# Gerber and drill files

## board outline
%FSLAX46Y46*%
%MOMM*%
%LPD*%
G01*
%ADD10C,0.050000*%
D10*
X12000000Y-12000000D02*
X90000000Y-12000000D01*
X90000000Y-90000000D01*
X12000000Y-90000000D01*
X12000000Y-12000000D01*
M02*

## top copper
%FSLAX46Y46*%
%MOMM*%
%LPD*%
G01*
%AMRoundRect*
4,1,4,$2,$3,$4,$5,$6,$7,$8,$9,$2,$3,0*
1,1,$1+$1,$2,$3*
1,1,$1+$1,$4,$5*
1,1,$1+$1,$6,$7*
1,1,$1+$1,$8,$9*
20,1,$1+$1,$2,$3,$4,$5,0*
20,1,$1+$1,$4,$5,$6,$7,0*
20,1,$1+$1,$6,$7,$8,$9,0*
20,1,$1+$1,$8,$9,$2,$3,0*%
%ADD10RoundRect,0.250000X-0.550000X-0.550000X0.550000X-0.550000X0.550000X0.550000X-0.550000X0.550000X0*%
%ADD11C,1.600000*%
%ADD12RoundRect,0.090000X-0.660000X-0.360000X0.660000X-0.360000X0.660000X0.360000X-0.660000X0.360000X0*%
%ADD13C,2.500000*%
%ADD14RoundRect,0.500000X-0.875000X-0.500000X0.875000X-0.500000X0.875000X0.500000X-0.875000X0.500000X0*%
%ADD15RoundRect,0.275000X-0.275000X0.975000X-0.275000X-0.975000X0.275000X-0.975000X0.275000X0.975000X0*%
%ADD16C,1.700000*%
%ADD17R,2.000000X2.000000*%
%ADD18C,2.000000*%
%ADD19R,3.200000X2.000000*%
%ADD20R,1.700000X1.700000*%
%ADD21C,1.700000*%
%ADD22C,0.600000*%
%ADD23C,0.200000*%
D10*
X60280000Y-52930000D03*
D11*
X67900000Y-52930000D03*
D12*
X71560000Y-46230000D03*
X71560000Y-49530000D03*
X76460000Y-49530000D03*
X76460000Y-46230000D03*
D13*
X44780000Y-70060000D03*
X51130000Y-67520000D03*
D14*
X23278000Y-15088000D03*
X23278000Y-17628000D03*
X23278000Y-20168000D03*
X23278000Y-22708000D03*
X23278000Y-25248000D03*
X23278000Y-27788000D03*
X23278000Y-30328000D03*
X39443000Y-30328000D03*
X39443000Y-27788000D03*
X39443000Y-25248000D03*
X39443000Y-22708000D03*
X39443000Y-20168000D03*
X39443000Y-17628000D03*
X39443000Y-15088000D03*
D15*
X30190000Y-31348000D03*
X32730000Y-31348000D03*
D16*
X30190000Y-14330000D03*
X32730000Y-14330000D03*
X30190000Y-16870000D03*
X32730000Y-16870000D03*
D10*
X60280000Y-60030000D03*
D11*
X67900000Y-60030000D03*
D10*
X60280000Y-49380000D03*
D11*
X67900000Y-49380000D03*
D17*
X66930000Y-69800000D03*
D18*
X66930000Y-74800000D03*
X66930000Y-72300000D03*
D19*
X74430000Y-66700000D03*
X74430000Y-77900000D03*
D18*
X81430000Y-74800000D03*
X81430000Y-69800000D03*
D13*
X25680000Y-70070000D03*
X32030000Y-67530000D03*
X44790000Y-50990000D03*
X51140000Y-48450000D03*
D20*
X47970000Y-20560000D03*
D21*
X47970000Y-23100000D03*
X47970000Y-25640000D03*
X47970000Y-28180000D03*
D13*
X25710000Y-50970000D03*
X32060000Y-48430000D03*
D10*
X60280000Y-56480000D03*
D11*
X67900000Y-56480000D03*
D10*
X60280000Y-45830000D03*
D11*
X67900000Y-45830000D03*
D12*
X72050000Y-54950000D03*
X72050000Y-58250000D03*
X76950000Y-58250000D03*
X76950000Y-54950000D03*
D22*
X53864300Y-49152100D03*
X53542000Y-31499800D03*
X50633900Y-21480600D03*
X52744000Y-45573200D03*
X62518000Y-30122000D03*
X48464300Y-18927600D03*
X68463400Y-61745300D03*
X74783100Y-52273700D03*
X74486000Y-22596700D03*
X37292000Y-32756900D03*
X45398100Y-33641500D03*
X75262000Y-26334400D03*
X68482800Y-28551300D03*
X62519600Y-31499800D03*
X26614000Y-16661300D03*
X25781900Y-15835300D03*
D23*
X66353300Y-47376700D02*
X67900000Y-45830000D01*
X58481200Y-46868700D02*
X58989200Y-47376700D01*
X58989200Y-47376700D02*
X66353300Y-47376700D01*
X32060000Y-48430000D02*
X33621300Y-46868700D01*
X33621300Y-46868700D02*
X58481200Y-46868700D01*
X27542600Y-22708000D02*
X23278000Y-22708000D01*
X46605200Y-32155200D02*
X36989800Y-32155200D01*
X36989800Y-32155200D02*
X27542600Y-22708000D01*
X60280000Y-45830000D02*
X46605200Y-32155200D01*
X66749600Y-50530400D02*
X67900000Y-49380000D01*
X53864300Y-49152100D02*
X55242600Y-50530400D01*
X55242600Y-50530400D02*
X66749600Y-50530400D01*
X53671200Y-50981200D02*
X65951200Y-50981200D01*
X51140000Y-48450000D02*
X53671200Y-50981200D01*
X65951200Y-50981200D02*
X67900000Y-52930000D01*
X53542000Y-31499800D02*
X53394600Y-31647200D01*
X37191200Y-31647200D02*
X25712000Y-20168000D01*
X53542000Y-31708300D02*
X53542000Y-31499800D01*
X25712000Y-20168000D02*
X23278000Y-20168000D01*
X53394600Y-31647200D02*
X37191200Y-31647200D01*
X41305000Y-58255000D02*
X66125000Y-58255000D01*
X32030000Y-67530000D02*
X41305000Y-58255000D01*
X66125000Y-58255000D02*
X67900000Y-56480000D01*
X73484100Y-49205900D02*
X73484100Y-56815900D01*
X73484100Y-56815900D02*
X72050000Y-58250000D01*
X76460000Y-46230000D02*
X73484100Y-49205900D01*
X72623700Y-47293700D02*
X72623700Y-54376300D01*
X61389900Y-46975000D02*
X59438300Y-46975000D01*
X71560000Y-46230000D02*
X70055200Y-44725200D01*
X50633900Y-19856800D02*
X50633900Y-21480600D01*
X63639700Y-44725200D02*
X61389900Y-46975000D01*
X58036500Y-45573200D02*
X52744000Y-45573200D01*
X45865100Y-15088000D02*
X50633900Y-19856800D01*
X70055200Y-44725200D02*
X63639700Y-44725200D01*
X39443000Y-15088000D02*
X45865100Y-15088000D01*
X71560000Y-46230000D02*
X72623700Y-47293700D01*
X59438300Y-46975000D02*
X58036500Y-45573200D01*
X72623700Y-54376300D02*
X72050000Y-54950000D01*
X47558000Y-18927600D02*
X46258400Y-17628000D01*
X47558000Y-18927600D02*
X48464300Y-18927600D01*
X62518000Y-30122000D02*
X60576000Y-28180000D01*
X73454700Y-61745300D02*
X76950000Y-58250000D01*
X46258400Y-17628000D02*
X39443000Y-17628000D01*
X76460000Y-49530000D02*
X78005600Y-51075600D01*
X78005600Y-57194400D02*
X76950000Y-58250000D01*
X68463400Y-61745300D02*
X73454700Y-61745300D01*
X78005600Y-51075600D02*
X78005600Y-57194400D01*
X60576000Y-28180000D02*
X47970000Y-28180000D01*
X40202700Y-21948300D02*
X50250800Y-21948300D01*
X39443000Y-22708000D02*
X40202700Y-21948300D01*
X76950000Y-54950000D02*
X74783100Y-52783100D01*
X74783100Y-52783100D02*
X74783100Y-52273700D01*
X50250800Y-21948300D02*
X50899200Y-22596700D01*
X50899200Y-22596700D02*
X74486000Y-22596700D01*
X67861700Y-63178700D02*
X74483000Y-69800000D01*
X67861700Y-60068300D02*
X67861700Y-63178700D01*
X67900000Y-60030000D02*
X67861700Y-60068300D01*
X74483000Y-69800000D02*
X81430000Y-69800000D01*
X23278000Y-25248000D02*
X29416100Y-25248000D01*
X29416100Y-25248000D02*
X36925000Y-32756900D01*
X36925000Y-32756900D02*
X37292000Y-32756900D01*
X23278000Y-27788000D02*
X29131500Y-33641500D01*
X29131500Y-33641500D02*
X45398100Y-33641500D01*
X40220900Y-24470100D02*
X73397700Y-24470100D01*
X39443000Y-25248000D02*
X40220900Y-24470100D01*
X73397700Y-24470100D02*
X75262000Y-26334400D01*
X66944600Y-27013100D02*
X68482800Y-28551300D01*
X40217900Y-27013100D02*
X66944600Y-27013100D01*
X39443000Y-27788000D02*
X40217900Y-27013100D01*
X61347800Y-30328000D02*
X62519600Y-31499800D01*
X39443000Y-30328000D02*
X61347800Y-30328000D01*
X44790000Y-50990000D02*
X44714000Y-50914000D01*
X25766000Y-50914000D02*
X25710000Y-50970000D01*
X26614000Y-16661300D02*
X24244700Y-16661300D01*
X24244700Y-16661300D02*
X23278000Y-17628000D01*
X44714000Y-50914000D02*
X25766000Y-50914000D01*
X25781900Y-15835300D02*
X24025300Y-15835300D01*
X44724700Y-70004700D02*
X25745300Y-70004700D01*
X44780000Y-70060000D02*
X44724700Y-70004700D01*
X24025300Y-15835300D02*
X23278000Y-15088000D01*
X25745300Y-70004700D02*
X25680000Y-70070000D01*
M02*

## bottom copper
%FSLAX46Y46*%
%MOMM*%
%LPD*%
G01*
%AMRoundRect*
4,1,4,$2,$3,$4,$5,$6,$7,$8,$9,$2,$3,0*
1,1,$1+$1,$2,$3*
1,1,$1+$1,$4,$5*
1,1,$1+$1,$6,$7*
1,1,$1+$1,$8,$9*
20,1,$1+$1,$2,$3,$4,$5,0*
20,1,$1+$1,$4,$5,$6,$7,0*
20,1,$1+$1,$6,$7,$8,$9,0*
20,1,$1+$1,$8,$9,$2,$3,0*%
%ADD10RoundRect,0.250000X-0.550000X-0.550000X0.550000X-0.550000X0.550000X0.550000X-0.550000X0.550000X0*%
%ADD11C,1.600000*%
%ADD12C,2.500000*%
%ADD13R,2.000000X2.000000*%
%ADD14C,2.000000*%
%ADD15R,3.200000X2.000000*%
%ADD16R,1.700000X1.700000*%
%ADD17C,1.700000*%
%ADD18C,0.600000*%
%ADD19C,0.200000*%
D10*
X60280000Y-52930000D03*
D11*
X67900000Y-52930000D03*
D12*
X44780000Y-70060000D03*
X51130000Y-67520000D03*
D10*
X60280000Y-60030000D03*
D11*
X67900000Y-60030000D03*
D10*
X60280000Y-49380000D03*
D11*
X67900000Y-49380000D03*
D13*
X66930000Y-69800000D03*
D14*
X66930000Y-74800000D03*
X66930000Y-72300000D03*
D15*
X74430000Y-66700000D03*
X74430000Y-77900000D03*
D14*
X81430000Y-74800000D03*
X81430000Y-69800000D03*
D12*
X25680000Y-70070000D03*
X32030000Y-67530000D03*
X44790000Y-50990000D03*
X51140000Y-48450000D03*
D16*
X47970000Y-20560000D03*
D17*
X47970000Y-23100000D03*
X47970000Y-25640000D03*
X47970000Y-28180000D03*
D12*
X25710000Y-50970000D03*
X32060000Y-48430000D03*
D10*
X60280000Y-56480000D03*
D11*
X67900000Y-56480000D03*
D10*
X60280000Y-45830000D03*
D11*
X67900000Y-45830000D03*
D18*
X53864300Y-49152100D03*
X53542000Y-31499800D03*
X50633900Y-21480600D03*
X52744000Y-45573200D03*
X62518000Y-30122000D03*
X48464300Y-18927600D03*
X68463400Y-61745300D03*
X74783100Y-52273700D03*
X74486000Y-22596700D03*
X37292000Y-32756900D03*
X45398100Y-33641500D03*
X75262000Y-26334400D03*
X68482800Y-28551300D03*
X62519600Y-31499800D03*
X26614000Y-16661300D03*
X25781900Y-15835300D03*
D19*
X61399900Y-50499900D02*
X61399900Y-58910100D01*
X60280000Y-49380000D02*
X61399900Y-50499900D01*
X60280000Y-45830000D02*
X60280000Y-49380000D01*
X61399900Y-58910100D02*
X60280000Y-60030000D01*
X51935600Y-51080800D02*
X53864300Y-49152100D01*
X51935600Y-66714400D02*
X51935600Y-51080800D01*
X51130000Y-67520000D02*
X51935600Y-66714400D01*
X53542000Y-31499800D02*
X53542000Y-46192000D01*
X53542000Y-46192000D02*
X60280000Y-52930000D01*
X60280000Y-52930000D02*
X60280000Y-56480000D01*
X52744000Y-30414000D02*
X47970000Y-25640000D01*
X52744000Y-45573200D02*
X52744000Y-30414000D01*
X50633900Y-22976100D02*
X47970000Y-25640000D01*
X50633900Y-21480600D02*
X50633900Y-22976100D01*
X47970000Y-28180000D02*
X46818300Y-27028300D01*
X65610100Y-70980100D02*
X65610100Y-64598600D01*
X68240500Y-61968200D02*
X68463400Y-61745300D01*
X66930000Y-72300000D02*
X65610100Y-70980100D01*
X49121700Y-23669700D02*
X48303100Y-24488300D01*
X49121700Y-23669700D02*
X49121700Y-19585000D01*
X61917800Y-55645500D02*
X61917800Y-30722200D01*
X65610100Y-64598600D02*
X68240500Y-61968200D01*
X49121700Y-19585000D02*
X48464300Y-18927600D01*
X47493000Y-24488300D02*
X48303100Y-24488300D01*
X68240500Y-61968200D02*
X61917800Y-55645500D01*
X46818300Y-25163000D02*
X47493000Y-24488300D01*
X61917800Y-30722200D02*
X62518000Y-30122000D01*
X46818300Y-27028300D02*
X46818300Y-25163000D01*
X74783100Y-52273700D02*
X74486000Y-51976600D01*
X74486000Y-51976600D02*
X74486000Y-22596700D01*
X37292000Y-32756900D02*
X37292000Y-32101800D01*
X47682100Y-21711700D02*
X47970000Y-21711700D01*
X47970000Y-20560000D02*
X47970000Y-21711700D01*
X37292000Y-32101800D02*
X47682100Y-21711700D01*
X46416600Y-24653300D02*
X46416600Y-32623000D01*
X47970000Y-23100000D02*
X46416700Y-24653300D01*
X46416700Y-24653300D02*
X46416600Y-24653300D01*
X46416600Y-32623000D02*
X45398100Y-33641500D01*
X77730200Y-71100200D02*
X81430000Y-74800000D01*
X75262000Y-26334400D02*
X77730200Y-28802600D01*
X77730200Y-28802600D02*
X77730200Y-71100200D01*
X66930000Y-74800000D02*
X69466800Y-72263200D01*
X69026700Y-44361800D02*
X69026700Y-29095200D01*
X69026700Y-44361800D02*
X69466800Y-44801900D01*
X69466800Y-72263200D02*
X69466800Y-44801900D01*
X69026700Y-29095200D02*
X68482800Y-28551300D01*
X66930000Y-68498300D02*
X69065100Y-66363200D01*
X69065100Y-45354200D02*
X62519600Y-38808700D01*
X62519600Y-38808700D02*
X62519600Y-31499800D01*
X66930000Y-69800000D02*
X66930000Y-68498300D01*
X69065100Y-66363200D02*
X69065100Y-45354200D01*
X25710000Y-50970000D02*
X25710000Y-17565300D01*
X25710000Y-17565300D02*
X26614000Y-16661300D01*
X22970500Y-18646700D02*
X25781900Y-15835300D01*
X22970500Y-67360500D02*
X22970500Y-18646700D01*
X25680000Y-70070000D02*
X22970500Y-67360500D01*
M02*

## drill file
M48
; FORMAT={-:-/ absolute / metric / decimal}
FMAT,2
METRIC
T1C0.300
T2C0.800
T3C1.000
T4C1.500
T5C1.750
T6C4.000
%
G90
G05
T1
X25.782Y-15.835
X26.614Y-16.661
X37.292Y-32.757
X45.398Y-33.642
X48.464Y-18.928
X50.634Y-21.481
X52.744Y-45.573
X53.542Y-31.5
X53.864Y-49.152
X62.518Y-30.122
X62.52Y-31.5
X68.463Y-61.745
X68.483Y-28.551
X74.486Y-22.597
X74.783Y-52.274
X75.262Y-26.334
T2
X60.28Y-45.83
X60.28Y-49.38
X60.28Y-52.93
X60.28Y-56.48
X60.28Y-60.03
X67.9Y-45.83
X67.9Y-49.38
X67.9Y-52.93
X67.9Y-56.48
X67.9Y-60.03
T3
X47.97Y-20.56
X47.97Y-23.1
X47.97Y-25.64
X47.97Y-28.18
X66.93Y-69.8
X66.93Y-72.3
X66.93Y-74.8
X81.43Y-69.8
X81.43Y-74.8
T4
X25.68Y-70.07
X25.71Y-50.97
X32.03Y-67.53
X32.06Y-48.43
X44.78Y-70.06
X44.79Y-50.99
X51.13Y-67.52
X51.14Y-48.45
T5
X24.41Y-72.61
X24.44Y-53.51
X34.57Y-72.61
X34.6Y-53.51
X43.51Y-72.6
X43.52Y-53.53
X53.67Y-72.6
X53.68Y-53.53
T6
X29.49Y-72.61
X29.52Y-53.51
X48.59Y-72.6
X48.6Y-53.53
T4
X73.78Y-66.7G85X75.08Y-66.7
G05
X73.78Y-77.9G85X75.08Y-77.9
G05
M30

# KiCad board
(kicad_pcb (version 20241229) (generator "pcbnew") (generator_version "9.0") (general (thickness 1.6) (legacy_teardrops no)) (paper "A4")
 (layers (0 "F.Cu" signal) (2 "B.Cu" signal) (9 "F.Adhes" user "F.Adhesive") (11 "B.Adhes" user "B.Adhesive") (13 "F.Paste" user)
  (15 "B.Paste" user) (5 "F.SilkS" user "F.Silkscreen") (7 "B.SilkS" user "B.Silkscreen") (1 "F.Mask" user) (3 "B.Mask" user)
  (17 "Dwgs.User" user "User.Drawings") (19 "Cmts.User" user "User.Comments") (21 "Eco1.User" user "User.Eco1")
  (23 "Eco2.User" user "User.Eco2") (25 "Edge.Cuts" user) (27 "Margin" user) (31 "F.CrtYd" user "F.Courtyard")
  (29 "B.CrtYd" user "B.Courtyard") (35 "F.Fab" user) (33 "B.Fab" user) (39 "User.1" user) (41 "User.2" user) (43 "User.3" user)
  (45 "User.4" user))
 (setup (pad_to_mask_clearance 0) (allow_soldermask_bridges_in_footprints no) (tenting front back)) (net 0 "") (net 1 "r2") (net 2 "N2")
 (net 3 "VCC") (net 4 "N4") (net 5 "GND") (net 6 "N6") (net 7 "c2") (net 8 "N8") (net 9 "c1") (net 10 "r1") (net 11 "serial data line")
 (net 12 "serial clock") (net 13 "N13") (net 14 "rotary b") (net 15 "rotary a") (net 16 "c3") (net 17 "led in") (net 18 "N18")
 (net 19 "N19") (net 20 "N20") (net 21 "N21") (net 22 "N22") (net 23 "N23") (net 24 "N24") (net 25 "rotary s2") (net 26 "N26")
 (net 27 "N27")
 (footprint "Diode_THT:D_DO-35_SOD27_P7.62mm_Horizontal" (layer "F.Cu") (at 60.28 52.93)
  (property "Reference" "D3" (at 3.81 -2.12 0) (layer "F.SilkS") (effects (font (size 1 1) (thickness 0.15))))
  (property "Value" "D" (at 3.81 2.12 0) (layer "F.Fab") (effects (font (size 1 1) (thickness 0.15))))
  (pad "1" thru_hole roundrect (at 0 0) (size 1.6 1.6) (drill 0.8) (layers "*.Cu" "*.Mask") (remove_unused_layers no)
   (roundrect_rratio 0.15625) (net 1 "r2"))
  (pad "2" thru_hole circle (at 7.62 0) (size 1.6 1.6) (drill 0.8) (layers "*.Cu" "*.Mask") (remove_unused_layers no) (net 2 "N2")))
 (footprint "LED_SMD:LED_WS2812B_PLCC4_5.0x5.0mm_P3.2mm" (layer "F.Cu") (at 74.01 47.88)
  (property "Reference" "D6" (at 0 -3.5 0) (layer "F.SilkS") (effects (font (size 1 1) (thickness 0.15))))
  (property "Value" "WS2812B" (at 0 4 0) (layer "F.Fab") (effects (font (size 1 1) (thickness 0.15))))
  (pad "1" smd roundrect (at -2.45 -1.65) (size 1.5 0.9) (layers "F.Cu" "F.Mask" "F.Paste") (roundrect_rratio 0.1) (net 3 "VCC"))
  (pad "2" smd roundrect (at -2.45 1.65) (size 1.5 0.9) (layers "F.Cu" "F.Mask" "F.Paste") (roundrect_rratio 0.1) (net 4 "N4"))
  (pad "3" smd roundrect (at 2.45 1.65) (size 1.5 0.9) (layers "F.Cu" "F.Mask" "F.Paste") (roundrect_rratio 0.1) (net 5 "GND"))
  (pad "4" smd roundrect (at 2.45 -1.65) (size 1.5 0.9) (layers "F.Cu" "F.Mask" "F.Paste") (roundrect_rratio 0.1) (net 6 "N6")))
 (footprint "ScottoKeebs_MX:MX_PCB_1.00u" (layer "F.Cu") (at 48.59 72.6)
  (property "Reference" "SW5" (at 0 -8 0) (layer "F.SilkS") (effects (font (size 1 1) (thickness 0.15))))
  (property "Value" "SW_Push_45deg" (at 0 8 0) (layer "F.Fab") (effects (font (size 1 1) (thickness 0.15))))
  (pad "" np_thru_hole circle (at -5.08 0) (size 1.75 1.75) (drill 1.75) (layers "*.Cu" "*.Mask"))
  (pad "" np_thru_hole circle (at 0 0) (size 4 4) (drill 4) (layers "*.Cu" "*.Mask"))
  (pad "" np_thru_hole circle (at 5.08 0) (size 1.75 1.75) (drill 1.75) (layers "*.Cu" "*.Mask"))
  (pad "1" thru_hole circle (at -3.81 -2.54) (size 2.5 2.5) (drill 1.5) (layers "*.Cu" "*.Mask") (remove_unused_layers no) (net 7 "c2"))
  (pad "2" thru_hole circle (at 2.54 -5.08) (size 2.5 2.5) (drill 1.5) (layers "*.Cu" "*.Mask") (remove_unused_layers no) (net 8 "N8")))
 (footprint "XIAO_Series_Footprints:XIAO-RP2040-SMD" (layer "F.Cu") (at 22.443 33.208)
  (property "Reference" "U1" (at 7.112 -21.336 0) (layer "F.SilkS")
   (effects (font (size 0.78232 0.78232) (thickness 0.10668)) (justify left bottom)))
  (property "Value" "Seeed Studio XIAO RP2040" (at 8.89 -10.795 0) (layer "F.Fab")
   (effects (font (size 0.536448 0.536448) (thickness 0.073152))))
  (pad "1" smd roundrect (at 0.835 -18.12) (size 2.75 2) (layers "F.Cu" "F.Mask" "F.Paste") (roundrect_rratio 0.25) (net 7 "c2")
   (solder_mask_margin 0.0508) (thermal_bridge_angle 45))
  (pad "2" smd roundrect (at 0.835 -15.58) (size 2.75 2) (layers "F.Cu" "F.Mask" "F.Paste") (roundrect_rratio 0.25) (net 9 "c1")
   (solder_mask_margin 0.0508) (thermal_bridge_angle 45))
  (pad "3" smd roundrect (at 0.835 -13.04) (size 2.75 2) (layers "F.Cu" "F.Mask" "F.Paste") (roundrect_rratio 0.25) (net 1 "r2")
   (solder_mask_margin 0.0508) (thermal_bridge_angle 45))
  (pad "4" smd roundrect (at 0.835 -10.5) (size 2.75 2) (layers "F.Cu" "F.Mask" "F.Paste") (roundrect_rratio 0.25) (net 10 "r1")
   (solder_mask_margin 0.0508) (thermal_bridge_angle 45))
  (pad "5" smd roundrect (at 0.835 -7.96) (size 2.75 2) (layers "F.Cu" "F.Mask" "F.Paste") (roundrect_rratio 0.25)
   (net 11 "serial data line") (solder_mask_margin 0.0508) (thermal_bridge_angle 45))
  (pad "6" smd roundrect (at 0.835 -5.42) (size 2.75 2) (layers "F.Cu" "F.Mask" "F.Paste") (roundrect_rratio 0.25) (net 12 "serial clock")
   (solder_mask_margin 0.0508) (thermal_bridge_angle 45))
  (pad "7" smd roundrect (at 0.835 -2.88) (size 2.75 2) (layers "F.Cu" "F.Mask" "F.Paste") (roundrect_rratio 0.25) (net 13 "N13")
   (solder_mask_margin 0.0508) (thermal_bridge_angle 45))
  (pad "8" smd roundrect (at 17 -2.88) (size 2.75 2) (layers "F.Cu" "F.Mask" "F.Paste") (roundrect_rratio 0.25) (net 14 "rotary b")
   (solder_mask_margin 0.0508) (thermal_bridge_angle 45))
  (pad "9" smd roundrect (at 17 -5.42) (size 2.75 2) (layers "F.Cu" "F.Mask" "F.Paste") (roundrect_rratio 0.25) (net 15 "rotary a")
   (solder_mask_margin 0.0508) (thermal_bridge_angle 45))
  (pad "10" smd roundrect (at 17 -7.96) (size 2.75 2) (layers "F.Cu" "F.Mask" "F.Paste") (roundrect_rratio 0.25) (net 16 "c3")
   (solder_mask_margin 0.0508) (thermal_bridge_angle 45))
  (pad "11" smd roundrect (at 17 -10.5) (size 2.75 2) (layers "F.Cu" "F.Mask" "F.Paste") (roundrect_rratio 0.25) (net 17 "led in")
   (solder_mask_margin 0.0508) (thermal_bridge_angle 45))
  (pad "12" smd roundrect (at 17 -13.04) (size 2.75 2) (layers "F.Cu" "F.Mask" "F.Paste") (roundrect_rratio 0.25) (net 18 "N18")
   (solder_mask_margin 0.0508) (thermal_bridge_angle 45))
  (pad "13" smd roundrect (at 17 -15.58) (size 2.75 2) (layers "F.Cu" "F.Mask" "F.Paste") (roundrect_rratio 0.25) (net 5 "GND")
   (solder_mask_margin 0.0508) (thermal_bridge_angle 45))
  (pad "14" smd roundrect (at 17 -18.12) (size 2.75 2) (layers "F.Cu" "F.Mask" "F.Paste") (roundrect_rratio 0.25) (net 3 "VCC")
   (solder_mask_margin 0.0508) (thermal_bridge_angle 45))
  (pad "15" smd roundrect (at 7.747 -1.86 270) (size 2.5 1.1) (layers "F.Cu" "F.Mask" "F.Paste") (roundrect_rratio 0.25) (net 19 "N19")
   (thermal_bridge_angle 45))
  (pad "16" smd roundrect (at 10.287 -1.86 270) (size 2.5 1.1) (layers "F.Cu" "F.Mask" "F.Paste") (roundrect_rratio 0.25) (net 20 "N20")
   (thermal_bridge_angle 45))
  (pad "17" smd circle (at 7.747 -18.878) (size 1.7 1.7) (layers "F.Cu" "F.Mask" "F.Paste") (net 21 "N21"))
  (pad "18" smd circle (at 10.287 -18.878) (size 1.7 1.7) (layers "F.Cu" "F.Mask" "F.Paste") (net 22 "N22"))
  (pad "19" smd circle (at 7.747 -16.338) (size 1.7 1.7) (layers "F.Cu" "F.Mask" "F.Paste") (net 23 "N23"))
  (pad "20" smd circle (at 10.287 -16.338) (size 1.7 1.7) (layers "F.Cu" "F.Mask" "F.Paste") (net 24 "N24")))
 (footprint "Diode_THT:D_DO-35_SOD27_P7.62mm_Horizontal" (layer "F.Cu") (at 60.28 60.03)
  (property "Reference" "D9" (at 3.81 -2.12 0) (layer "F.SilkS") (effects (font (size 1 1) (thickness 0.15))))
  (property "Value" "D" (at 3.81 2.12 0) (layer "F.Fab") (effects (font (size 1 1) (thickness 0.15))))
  (pad "1" thru_hole roundrect (at 0 0) (size 1.6 1.6) (drill 0.8) (layers "*.Cu" "*.Mask") (remove_unused_layers no)
   (roundrect_rratio 0.15625) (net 10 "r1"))
  (pad "2" thru_hole circle (at 7.62 0) (size 1.6 1.6) (drill 0.8) (layers "*.Cu" "*.Mask") (remove_unused_layers no) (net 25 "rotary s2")))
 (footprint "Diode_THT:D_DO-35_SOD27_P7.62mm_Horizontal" (layer "F.Cu") (at 60.28 49.38)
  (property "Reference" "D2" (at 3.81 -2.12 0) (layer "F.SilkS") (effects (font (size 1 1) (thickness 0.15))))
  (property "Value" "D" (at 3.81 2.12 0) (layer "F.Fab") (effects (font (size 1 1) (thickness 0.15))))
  (pad "1" thru_hole roundrect (at 0 0) (size 1.6 1.6) (drill 0.8) (layers "*.Cu" "*.Mask") (remove_unused_layers no)
   (roundrect_rratio 0.15625) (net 10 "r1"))
  (pad "2" thru_hole circle (at 7.62 0) (size 1.6 1.6) (drill 0.8) (layers "*.Cu" "*.Mask") (remove_unused_layers no) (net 8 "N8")))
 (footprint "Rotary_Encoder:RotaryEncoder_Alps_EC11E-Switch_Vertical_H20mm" (layer "F.Cu") (at 66.93 69.8)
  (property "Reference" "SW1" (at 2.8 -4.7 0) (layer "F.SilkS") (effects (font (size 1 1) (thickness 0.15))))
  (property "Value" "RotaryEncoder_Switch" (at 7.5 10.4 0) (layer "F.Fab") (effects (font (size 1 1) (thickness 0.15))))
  (pad "A" thru_hole rect (at 0 0) (size 2 2) (drill 1) (layers "*.Cu" "*.Mask") (remove_unused_layers no) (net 14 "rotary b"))
  (pad "B" thru_hole circle (at 0 5) (size 2 2) (drill 1) (layers "*.Cu" "*.Mask") (remove_unused_layers no) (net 15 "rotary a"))
  (pad "C" thru_hole circle (at 0 2.5) (size 2 2) (drill 1) (layers "*.Cu" "*.Mask") (remove_unused_layers no) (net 5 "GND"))
  (pad "MP" thru_hole rect (at 7.5 -3.1) (size 3.2 2) (drill oval 2.8 1.5) (layers "*.Cu" "*.Mask") (remove_unused_layers no))
  (pad "MP" thru_hole rect (at 7.5 8.1) (size 3.2 2) (drill oval 2.8 1.5) (layers "*.Cu" "*.Mask") (remove_unused_layers no))
  (pad "S1" thru_hole circle (at 14.5 5) (size 2 2) (drill 1) (layers "*.Cu" "*.Mask") (remove_unused_layers no) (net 16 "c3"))
  (pad "S2" thru_hole circle (at 14.5 0) (size 2 2) (drill 1) (layers "*.Cu" "*.Mask") (remove_unused_layers no) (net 25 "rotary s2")))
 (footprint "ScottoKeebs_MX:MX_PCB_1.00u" (layer "F.Cu") (at 29.49 72.61)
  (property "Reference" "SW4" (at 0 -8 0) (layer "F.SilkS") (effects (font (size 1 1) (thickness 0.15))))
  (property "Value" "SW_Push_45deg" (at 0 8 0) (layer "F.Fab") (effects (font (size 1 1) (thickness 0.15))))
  (pad "" np_thru_hole circle (at -5.08 0) (size 1.75 1.75) (drill 1.75) (layers "*.Cu" "*.Mask"))
  (pad "" np_thru_hole circle (at 0 0) (size 4 4) (drill 4) (layers "*.Cu" "*.Mask"))
  (pad "" np_thru_hole circle (at 5.08 0) (size 1.75 1.75) (drill 1.75) (layers "*.Cu" "*.Mask"))
  (pad "1" thru_hole circle (at -3.81 -2.54) (size 2.5 2.5) (drill 1.5) (layers "*.Cu" "*.Mask") (remove_unused_layers no) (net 7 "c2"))
  (pad "2" thru_hole circle (at 2.54 -5.08) (size 2.5 2.5) (drill 1.5) (layers "*.Cu" "*.Mask") (remove_unused_layers no) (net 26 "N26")))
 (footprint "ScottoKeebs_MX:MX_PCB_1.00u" (layer "F.Cu") (at 48.6 53.53)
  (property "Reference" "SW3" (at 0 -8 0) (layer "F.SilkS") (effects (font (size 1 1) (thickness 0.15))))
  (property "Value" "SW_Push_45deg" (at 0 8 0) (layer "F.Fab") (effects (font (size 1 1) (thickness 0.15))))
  (pad "" np_thru_hole circle (at -5.08 0) (size 1.75 1.75) (drill 1.75) (layers "*.Cu" "*.Mask"))
  (pad "" np_thru_hole circle (at 0 0) (size 4 4) (drill 4) (layers "*.Cu" "*.Mask"))
  (pad "" np_thru_hole circle (at 5.08 0) (size 1.75 1.75) (drill 1.75) (layers "*.Cu" "*.Mask"))
  (pad "1" thru_hole circle (at -3.81 -2.54) (size 2.5 2.5) (drill 1.5) (layers "*.Cu" "*.Mask") (remove_unused_layers no) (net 9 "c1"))
  (pad "2" thru_hole circle (at 2.54 -5.08) (size 2.5 2.5) (drill 1.5) (layers "*.Cu" "*.Mask") (remove_unused_layers no) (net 2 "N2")))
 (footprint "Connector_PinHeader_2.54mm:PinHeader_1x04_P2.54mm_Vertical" (layer "F.Cu") (at 47.97 20.56)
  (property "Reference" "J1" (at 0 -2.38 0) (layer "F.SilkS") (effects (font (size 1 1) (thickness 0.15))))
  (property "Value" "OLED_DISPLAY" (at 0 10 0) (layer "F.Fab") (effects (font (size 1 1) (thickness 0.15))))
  (pad "1" thru_hole rect (at 0 0) (size 1.7 1.7) (drill 1) (layers "*.Cu" "*.Mask") (remove_unused_layers no) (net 11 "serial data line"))
  (pad "2" thru_hole circle (at 0 2.54) (size 1.7 1.7) (drill 1) (layers "*.Cu" "*.Mask") (remove_unused_layers no) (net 12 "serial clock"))
  (pad "3" thru_hole circle (at 0 5.08) (size 1.7 1.7) (drill 1) (layers "*.Cu" "*.Mask") (remove_unused_layers no) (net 3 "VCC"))
  (pad "4" thru_hole circle (at 0 7.62) (size 1.7 1.7) (drill 1) (layers "*.Cu" "*.Mask") (remove_unused_layers no) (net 5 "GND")))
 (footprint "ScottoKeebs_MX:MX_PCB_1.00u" (layer "F.Cu") (at 29.52 53.51)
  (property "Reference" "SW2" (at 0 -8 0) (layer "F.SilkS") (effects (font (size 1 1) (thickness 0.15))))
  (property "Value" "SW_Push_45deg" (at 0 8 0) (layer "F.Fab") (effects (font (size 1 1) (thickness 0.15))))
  (pad "" np_thru_hole circle (at -5.08 0) (size 1.75 1.75) (drill 1.75) (layers "*.Cu" "*.Mask"))
  (pad "" np_thru_hole circle (at 0 0) (size 4 4) (drill 4) (layers "*.Cu" "*.Mask"))
  (pad "" np_thru_hole circle (at 5.08 0) (size 1.75 1.75) (drill 1.75) (layers "*.Cu" "*.Mask"))
  (pad "1" thru_hole circle (at -3.81 -2.54) (size 2.5 2.5) (drill 1.5) (layers "*.Cu" "*.Mask") (remove_unused_layers no) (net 9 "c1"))
  (pad "2" thru_hole circle (at 2.54 -5.08) (size 2.5 2.5) (drill 1.5) (layers "*.Cu" "*.Mask") (remove_unused_layers no) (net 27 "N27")))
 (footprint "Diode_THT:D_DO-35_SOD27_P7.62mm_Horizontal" (layer "F.Cu") (at 60.28 56.48)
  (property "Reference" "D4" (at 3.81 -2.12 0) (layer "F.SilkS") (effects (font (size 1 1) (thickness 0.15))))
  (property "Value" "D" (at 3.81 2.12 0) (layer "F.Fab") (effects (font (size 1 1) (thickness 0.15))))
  (pad "1" thru_hole roundrect (at 0 0) (size 1.6 1.6) (drill 0.8) (layers "*.Cu" "*.Mask") (remove_unused_layers no)
   (roundrect_rratio 0.15625) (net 1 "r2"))
  (pad "2" thru_hole circle (at 7.62 0) (size 1.6 1.6) (drill 0.8) (layers "*.Cu" "*.Mask") (remove_unused_layers no) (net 26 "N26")))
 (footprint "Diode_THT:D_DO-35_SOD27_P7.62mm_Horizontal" (layer "F.Cu") (at 60.28 45.83)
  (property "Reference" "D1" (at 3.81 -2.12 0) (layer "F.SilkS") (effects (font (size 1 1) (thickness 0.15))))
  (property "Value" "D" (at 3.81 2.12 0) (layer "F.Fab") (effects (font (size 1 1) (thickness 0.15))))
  (pad "1" thru_hole roundrect (at 0 0) (size 1.6 1.6) (drill 0.8) (layers "*.Cu" "*.Mask") (remove_unused_layers no)
   (roundrect_rratio 0.15625) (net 10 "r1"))
  (pad "2" thru_hole circle (at 7.62 0) (size 1.6 1.6) (drill 0.8) (layers "*.Cu" "*.Mask") (remove_unused_layers no) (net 27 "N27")))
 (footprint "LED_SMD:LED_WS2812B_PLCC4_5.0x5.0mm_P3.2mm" (layer "F.Cu") (at 74.5 56.6)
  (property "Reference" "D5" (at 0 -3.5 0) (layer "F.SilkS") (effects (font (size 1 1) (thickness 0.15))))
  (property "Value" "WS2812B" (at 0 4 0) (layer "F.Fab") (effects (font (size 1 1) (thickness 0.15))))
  (pad "1" smd roundrect (at -2.45 -1.65) (size 1.5 0.9) (layers "F.Cu" "F.Mask" "F.Paste") (roundrect_rratio 0.1) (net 3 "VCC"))
  (pad "2" smd roundrect (at -2.45 1.65) (size 1.5 0.9) (layers "F.Cu" "F.Mask" "F.Paste") (roundrect_rratio 0.1) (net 6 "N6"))
  (pad "3" smd roundrect (at 2.45 1.65) (size 1.5 0.9) (layers "F.Cu" "F.Mask" "F.Paste") (roundrect_rratio 0.1) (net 5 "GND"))
  (pad "4" smd roundrect (at 2.45 -1.65) (size 1.5 0.9) (layers "F.Cu" "F.Mask" "F.Paste") (roundrect_rratio 0.1) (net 17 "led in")))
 (gr_rect (start 12 12) (end 90 90) (stroke (width 0.05) (type solid)) (fill no) (layer "Edge.Cuts"))
 (segment (start 66.3533 47.3767) (end 67.9 45.83) (width 0.2) (layer "F.Cu") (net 27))
 (segment (start 58.4812 46.8687) (end 58.9892 47.3767) (width 0.2) (layer "F.Cu") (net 27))
 (segment (start 58.9892 47.3767) (end 66.3533 47.3767) (width 0.2) (layer "F.Cu") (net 27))
 (segment (start 32.06 48.43) (end 33.6213 46.8687) (width 0.2) (layer "F.Cu") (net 27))
 (segment (start 33.6213 46.8687) (end 58.4812 46.8687) (width 0.2) (layer "F.Cu") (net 27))
 (segment (start 27.5426 22.708) (end 23.278 22.708) (width 0.2) (layer "F.Cu") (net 10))
 (segment (start 46.6052 32.1552) (end 36.9898 32.1552) (width 0.2) (layer "F.Cu") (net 10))
 (segment (start 36.9898 32.1552) (end 27.5426 22.708) (width 0.2) (layer "F.Cu") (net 10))
 (segment (start 60.28 45.83) (end 46.6052 32.1552) (width 0.2) (layer "F.Cu") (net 10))
 (segment (start 61.3999 50.4999) (end 61.3999 58.9101) (width 0.2) (layer "B.Cu") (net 10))
 (segment (start 60.28 49.38) (end 61.3999 50.4999) (width 0.2) (layer "B.Cu") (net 10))
 (segment (start 60.28 45.83) (end 60.28 49.38) (width 0.2) (layer "B.Cu") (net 10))
 (segment (start 61.3999 58.9101) (end 60.28 60.03) (width 0.2) (layer "B.Cu") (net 10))
 (segment (start 66.7496 50.5304) (end 67.9 49.38) (width 0.2) (layer "F.Cu") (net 8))
 (segment (start 53.8643 49.1521) (end 55.2426 50.5304) (width 0.2) (layer "F.Cu") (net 8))
 (segment (start 55.2426 50.5304) (end 66.7496 50.5304) (width 0.2) (layer "F.Cu") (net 8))
 (via (at 53.8643 49.1521) (size 0.6) (drill 0.3) (layers "F.Cu" "B.Cu") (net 8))
 (segment (start 51.9356 51.0808) (end 53.8643 49.1521) (width 0.2) (layer "B.Cu") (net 8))
 (segment (start 51.9356 66.7144) (end 51.9356 51.0808) (width 0.2) (layer "B.Cu") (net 8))
 (segment (start 51.13 67.52) (end 51.9356 66.7144) (width 0.2) (layer "B.Cu") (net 8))
 (segment (start 53.6712 50.9812) (end 65.9512 50.9812) (width 0.2) (layer "F.Cu") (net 2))
 (segment (start 51.14 48.45) (end 53.6712 50.9812) (width 0.2) (layer "F.Cu") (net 2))
 (segment (start 65.9512 50.9812) (end 67.9 52.93) (width 0.2) (layer "F.Cu") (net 2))
 (segment (start 53.542 31.4998) (end 53.3946 31.6472) (width 0.2) (layer "F.Cu") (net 1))
 (segment (start 37.1912 31.6472) (end 25.712 20.168) (width 0.2) (layer "F.Cu") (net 1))
 (segment (start 53.542 31.7083) (end 53.542 31.4998) (width 0.2) (layer "F.Cu") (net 1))
 (segment (start 25.712 20.168) (end 23.278 20.168) (width 0.2) (layer "F.Cu") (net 1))
 (segment (start 53.3946 31.6472) (end 37.1912 31.6472) (width 0.2) (layer "F.Cu") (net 1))
 (via (at 53.542 31.4998) (size 0.6) (drill 0.3) (layers "F.Cu" "B.Cu") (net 1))
 (segment (start 53.542 31.4998) (end 53.542 46.192) (width 0.2) (layer "B.Cu") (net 1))
 (segment (start 53.542 46.192) (end 60.28 52.93) (width 0.2) (layer "B.Cu") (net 1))
 (segment (start 60.28 52.93) (end 60.28 56.48) (width 0.2) (layer "B.Cu") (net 1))
 (segment (start 41.305 58.255) (end 66.125 58.255) (width 0.2) (layer "F.Cu") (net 26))
 (segment (start 32.03 67.53) (end 41.305 58.255) (width 0.2) (layer "F.Cu") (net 26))
 (segment (start 66.125 58.255) (end 67.9 56.48) (width 0.2) (layer "F.Cu") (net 26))
 (segment (start 73.4841 49.2059) (end 73.4841 56.8159) (width 0.2) (layer "F.Cu") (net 6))
 (segment (start 73.4841 56.8159) (end 72.05 58.25) (width 0.2) (layer "F.Cu") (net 6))
 (segment (start 76.46 46.23) (end 73.4841 49.2059) (width 0.2) (layer "F.Cu") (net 6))
 (segment (start 72.6237 47.2937) (end 72.6237 54.3763) (width 0.2) (layer "F.Cu") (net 3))
 (segment (start 61.3899 46.975) (end 59.4383 46.975) (width 0.2) (layer "F.Cu") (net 3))
 (segment (start 71.56 46.23) (end 70.0552 44.7252) (width 0.2) (layer "F.Cu") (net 3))
 (segment (start 50.6339 19.8568) (end 50.6339 21.4806) (width 0.2) (layer "F.Cu") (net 3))
 (segment (start 63.6397 44.7252) (end 61.3899 46.975) (width 0.2) (layer "F.Cu") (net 3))
 (segment (start 58.0365 45.5732) (end 52.744 45.5732) (width 0.2) (layer "F.Cu") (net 3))
 (segment (start 45.8651 15.088) (end 50.6339 19.8568) (width 0.2) (layer "F.Cu") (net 3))
 (segment (start 70.0552 44.7252) (end 63.6397 44.7252) (width 0.2) (layer "F.Cu") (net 3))
 (segment (start 39.443 15.088) (end 45.8651 15.088) (width 0.2) (layer "F.Cu") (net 3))
 (segment (start 71.56 46.23) (end 72.6237 47.2937) (width 0.2) (layer "F.Cu") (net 3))
 (segment (start 59.4383 46.975) (end 58.0365 45.5732) (width 0.2) (layer "F.Cu") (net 3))
 (segment (start 72.6237 54.3763) (end 72.05 54.95) (width 0.2) (layer "F.Cu") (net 3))
 (via (at 50.6339 21.4806) (size 0.6) (drill 0.3) (layers "F.Cu" "B.Cu") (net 3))
 (via (at 52.744 45.5732) (size 0.6) (drill 0.3) (layers "F.Cu" "B.Cu") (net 3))
 (segment (start 52.744 30.414) (end 47.97 25.64) (width 0.2) (layer "B.Cu") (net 3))
 (segment (start 52.744 45.5732) (end 52.744 30.414) (width 0.2) (layer "B.Cu") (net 3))
 (segment (start 50.6339 22.9761) (end 47.97 25.64) (width 0.2) (layer "B.Cu") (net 3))
 (segment (start 50.6339 21.4806) (end 50.6339 22.9761) (width 0.2) (layer "B.Cu") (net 3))
 (segment (start 47.558 18.9276) (end 46.2584 17.628) (width 0.2) (layer "F.Cu") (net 5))
 (segment (start 47.558 18.9276) (end 48.4643 18.9276) (width 0.2) (layer "F.Cu") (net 5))
 (segment (start 62.518 30.122) (end 60.576 28.18) (width 0.2) (layer "F.Cu") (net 5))
 (segment (start 73.4547 61.7453) (end 76.95 58.25) (width 0.2) (layer "F.Cu") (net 5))
 (segment (start 46.2584 17.628) (end 39.443 17.628) (width 0.2) (layer "F.Cu") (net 5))
 (segment (start 76.46 49.53) (end 78.0056 51.0756) (width 0.2) (layer "F.Cu") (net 5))
 (segment (start 78.0056 57.1944) (end 76.95 58.25) (width 0.2) (layer "F.Cu") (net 5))
 (segment (start 68.4634 61.7453) (end 73.4547 61.7453) (width 0.2) (layer "F.Cu") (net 5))
 (segment (start 78.0056 51.0756) (end 78.0056 57.1944) (width 0.2) (layer "F.Cu") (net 5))
 (segment (start 60.576 28.18) (end 47.97 28.18) (width 0.2) (layer "F.Cu") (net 5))
 (via (at 62.518 30.122) (size 0.6) (drill 0.3) (layers "F.Cu" "B.Cu") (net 5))
 (via (at 48.4643 18.9276) (size 0.6) (drill 0.3) (layers "F.Cu" "B.Cu") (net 5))
 (via (at 68.4634 61.7453) (size 0.6) (drill 0.3) (layers "F.Cu" "B.Cu") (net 5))
 (segment (start 47.97 28.18) (end 46.8183 27.0283) (width 0.2) (layer "B.Cu") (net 5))
 (segment (start 65.6101 70.9801) (end 65.6101 64.5986) (width 0.2) (layer "B.Cu") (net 5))
 (segment (start 68.2405 61.9682) (end 68.4634 61.7453) (width 0.2) (layer "B.Cu") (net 5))
 (segment (start 66.93 72.3) (end 65.6101 70.9801) (width 0.2) (layer "B.Cu") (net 5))
 (segment (start 49.1217 23.6697) (end 48.3031 24.4883) (width 0.2) (layer "B.Cu") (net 5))
 (segment (start 49.1217 23.6697) (end 49.1217 19.585) (width 0.2) (layer "B.Cu") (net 5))
 (segment (start 61.9178 55.6455) (end 61.9178 30.7222) (width 0.2) (layer "B.Cu") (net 5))
 (segment (start 65.6101 64.5986) (end 68.2405 61.9682) (width 0.2) (layer "B.Cu") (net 5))
 (segment (start 49.1217 19.585) (end 48.4643 18.9276) (width 0.2) (layer "B.Cu") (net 5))
 (segment (start 47.493 24.4883) (end 48.3031 24.4883) (width 0.2) (layer "B.Cu") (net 5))
 (segment (start 68.2405 61.9682) (end 61.9178 55.6455) (width 0.2) (layer "B.Cu") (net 5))
 (segment (start 46.8183 25.163) (end 47.493 24.4883) (width 0.2) (layer "B.Cu") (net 5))
 (segment (start 61.9178 30.7222) (end 62.518 30.122) (width 0.2) (layer "B.Cu") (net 5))
 (segment (start 46.8183 27.0283) (end 46.8183 25.163) (width 0.2) (layer "B.Cu") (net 5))
 (segment (start 40.2027 21.9483) (end 50.2508 21.9483) (width 0.2) (layer "F.Cu") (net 17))
 (segment (start 39.443 22.708) (end 40.2027 21.9483) (width 0.2) (layer "F.Cu") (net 17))
 (segment (start 76.95 54.95) (end 74.7831 52.7831) (width 0.2) (layer "F.Cu") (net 17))
 (segment (start 74.7831 52.7831) (end 74.7831 52.2737) (width 0.2) (layer "F.Cu") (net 17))
 (segment (start 50.2508 21.9483) (end 50.8992 22.5967) (width 0.2) (layer "F.Cu") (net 17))
 (segment (start 50.8992 22.5967) (end 74.486 22.5967) (width 0.2) (layer "F.Cu") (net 17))
 (via (at 74.7831 52.2737) (size 0.6) (drill 0.3) (layers "F.Cu" "B.Cu") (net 17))
 (via (at 74.486 22.5967) (size 0.6) (drill 0.3) (layers "F.Cu" "B.Cu") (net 17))
 (segment (start 74.7831 52.2737) (end 74.486 51.9766) (width 0.2) (layer "B.Cu") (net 17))
 (segment (start 74.486 51.9766) (end 74.486 22.5967) (width 0.2) (layer "B.Cu") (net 17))
 (segment (start 67.8617 63.1787) (end 74.483 69.8) (width 0.2) (layer "F.Cu") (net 25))
 (segment (start 67.8617 60.0683) (end 67.8617 63.1787) (width 0.2) (layer "F.Cu") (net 25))
 (segment (start 67.9 60.03) (end 67.8617 60.0683) (width 0.2) (layer "F.Cu") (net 25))
 (segment (start 74.483 69.8) (end 81.43 69.8) (width 0.2) (layer "F.Cu") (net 25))
 (segment (start 23.278 25.248) (end 29.4161 25.248) (width 0.2) (layer "F.Cu") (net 11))
 (segment (start 29.4161 25.248) (end 36.925 32.7569) (width 0.2) (layer "F.Cu") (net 11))
 (segment (start 36.925 32.7569) (end 37.292 32.7569) (width 0.2) (layer "F.Cu") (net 11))
 (via (at 37.292 32.7569) (size 0.6) (drill 0.3) (layers "F.Cu" "B.Cu") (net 11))
 (segment (start 37.292 32.7569) (end 37.292 32.1018) (width 0.2) (layer "B.Cu") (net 11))
 (segment (start 47.6821 21.7117) (end 47.97 21.7117) (width 0.2) (layer "B.Cu") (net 11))
 (segment (start 47.97 20.56) (end 47.97 21.7117) (width 0.2) (layer "B.Cu") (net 11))
 (segment (start 37.292 32.1018) (end 47.6821 21.7117) (width 0.2) (layer "B.Cu") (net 11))
 (segment (start 23.278 27.788) (end 29.1315 33.6415) (width 0.2) (layer "F.Cu") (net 12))
 (segment (start 29.1315 33.6415) (end 45.3981 33.6415) (width 0.2) (layer "F.Cu") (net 12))
 (via (at 45.3981 33.6415) (size 0.6) (drill 0.3) (layers "F.Cu" "B.Cu") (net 12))
 (segment (start 46.4166 24.6533) (end 46.4166 32.623) (width 0.2) (layer "B.Cu") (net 12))
 (segment (start 47.97 23.1) (end 46.4167 24.6533) (width 0.2) (layer "B.Cu") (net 12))
 (segment (start 46.4167 24.6533) (end 46.4166 24.6533) (width 0.2) (layer "B.Cu") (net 12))
 (segment (start 46.4166 32.623) (end 45.3981 33.6415) (width 0.2) (layer "B.Cu") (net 12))
 (segment (start 40.2209 24.4701) (end 73.3977 24.4701) (width 0.2) (layer "F.Cu") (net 16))
 (segment (start 39.443 25.248) (end 40.2209 24.4701) (width 0.2) (layer "F.Cu") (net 16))
 (segment (start 73.3977 24.4701) (end 75.262 26.3344) (width 0.2) (layer "F.Cu") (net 16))
 (via (at 75.262 26.3344) (size 0.6) (drill 0.3) (layers "F.Cu" "B.Cu") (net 16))
 (segment (start 77.7302 71.1002) (end 81.43 74.8) (width 0.2) (layer "B.Cu") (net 16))
 (segment (start 75.262 26.3344) (end 77.7302 28.8026) (width 0.2) (layer "B.Cu") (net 16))
 (segment (start 77.7302 28.8026) (end 77.7302 71.1002) (width 0.2) (layer "B.Cu") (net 16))
 (segment (start 66.9446 27.0131) (end 68.4828 28.5513) (width 0.2) (layer "F.Cu") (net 15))
 (segment (start 40.2179 27.0131) (end 66.9446 27.0131) (width 0.2) (layer "F.Cu") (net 15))
 (segment (start 39.443 27.788) (end 40.2179 27.0131) (width 0.2) (layer "F.Cu") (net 15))
 (via (at 68.4828 28.5513) (size 0.6) (drill 0.3) (layers "F.Cu" "B.Cu") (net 15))
 (segment (start 66.93 74.8) (end 69.4668 72.2632) (width 0.2) (layer "B.Cu") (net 15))
 (segment (start 69.0267 44.3618) (end 69.0267 29.0952) (width 0.2) (layer "B.Cu") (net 15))
 (segment (start 69.0267 44.3618) (end 69.4668 44.8019) (width 0.2) (layer "B.Cu") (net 15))
 (segment (start 69.4668 72.2632) (end 69.4668 44.8019) (width 0.2) (layer "B.Cu") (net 15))
 (segment (start 69.0267 29.0952) (end 68.4828 28.5513) (width 0.2) (layer "B.Cu") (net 15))
 (segment (start 61.3478 30.328) (end 62.5196 31.4998) (width 0.2) (layer "F.Cu") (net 14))
 (segment (start 39.443 30.328) (end 61.3478 30.328) (width 0.2) (layer "F.Cu") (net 14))
 (via (at 62.5196 31.4998) (size 0.6) (drill 0.3) (layers "F.Cu" "B.Cu") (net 14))
 (segment (start 66.93 68.4983) (end 69.0651 66.3632) (width 0.2) (layer "B.Cu") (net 14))
 (segment (start 69.0651 45.3542) (end 62.5196 38.8087) (width 0.2) (layer "B.Cu") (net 14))
 (segment (start 62.5196 38.8087) (end 62.5196 31.4998) (width 0.2) (layer "B.Cu") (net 14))
 (segment (start 66.93 69.8) (end 66.93 68.4983) (width 0.2) (layer "B.Cu") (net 14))
 (segment (start 69.0651 66.3632) (end 69.0651 45.3542) (width 0.2) (layer "B.Cu") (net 14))
 (segment (start 44.79 50.99) (end 44.714 50.914) (width 0.2) (layer "F.Cu") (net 9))
 (segment (start 25.766 50.914) (end 25.71 50.97) (width 0.2) (layer "F.Cu") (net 9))
 (segment (start 26.614 16.6613) (end 24.2447 16.6613) (width 0.2) (layer "F.Cu") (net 9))
 (segment (start 24.2447 16.6613) (end 23.278 17.628) (width 0.2) (layer "F.Cu") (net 9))
 (segment (start 44.714 50.914) (end 25.766 50.914) (width 0.2) (layer "F.Cu") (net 9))
 (via (at 26.614 16.6613) (size 0.6) (drill 0.3) (layers "F.Cu" "B.Cu") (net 9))
 (segment (start 25.71 50.97) (end 25.71 17.5653) (width 0.2) (layer "B.Cu") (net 9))
 (segment (start 25.71 17.5653) (end 26.614 16.6613) (width 0.2) (layer "B.Cu") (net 9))
 (segment (start 25.7819 15.8353) (end 24.0253 15.8353) (width 0.2) (layer "F.Cu") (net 7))
 (segment (start 44.7247 70.0047) (end 25.7453 70.0047) (width 0.2) (layer "F.Cu") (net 7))
 (segment (start 44.78 70.06) (end 44.7247 70.0047) (width 0.2) (layer "F.Cu") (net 7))
 (segment (start 24.0253 15.8353) (end 23.278 15.088) (width 0.2) (layer "F.Cu") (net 7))
 (segment (start 25.7453 70.0047) (end 25.68 70.07) (width 0.2) (layer "F.Cu") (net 7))
 (via (at 25.7819 15.8353) (size 0.6) (drill 0.3) (layers "F.Cu" "B.Cu") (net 7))
 (segment (start 22.9705 18.6467) (end 25.7819 15.8353) (width 0.2) (layer "B.Cu") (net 7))
 (segment (start 22.9705 67.3605) (end 22.9705 18.6467) (width 0.2) (layer "B.Cu") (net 7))
 (segment (start 25.68 70.07) (end 22.9705 67.3605) (width 0.2) (layer "B.Cu") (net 7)))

